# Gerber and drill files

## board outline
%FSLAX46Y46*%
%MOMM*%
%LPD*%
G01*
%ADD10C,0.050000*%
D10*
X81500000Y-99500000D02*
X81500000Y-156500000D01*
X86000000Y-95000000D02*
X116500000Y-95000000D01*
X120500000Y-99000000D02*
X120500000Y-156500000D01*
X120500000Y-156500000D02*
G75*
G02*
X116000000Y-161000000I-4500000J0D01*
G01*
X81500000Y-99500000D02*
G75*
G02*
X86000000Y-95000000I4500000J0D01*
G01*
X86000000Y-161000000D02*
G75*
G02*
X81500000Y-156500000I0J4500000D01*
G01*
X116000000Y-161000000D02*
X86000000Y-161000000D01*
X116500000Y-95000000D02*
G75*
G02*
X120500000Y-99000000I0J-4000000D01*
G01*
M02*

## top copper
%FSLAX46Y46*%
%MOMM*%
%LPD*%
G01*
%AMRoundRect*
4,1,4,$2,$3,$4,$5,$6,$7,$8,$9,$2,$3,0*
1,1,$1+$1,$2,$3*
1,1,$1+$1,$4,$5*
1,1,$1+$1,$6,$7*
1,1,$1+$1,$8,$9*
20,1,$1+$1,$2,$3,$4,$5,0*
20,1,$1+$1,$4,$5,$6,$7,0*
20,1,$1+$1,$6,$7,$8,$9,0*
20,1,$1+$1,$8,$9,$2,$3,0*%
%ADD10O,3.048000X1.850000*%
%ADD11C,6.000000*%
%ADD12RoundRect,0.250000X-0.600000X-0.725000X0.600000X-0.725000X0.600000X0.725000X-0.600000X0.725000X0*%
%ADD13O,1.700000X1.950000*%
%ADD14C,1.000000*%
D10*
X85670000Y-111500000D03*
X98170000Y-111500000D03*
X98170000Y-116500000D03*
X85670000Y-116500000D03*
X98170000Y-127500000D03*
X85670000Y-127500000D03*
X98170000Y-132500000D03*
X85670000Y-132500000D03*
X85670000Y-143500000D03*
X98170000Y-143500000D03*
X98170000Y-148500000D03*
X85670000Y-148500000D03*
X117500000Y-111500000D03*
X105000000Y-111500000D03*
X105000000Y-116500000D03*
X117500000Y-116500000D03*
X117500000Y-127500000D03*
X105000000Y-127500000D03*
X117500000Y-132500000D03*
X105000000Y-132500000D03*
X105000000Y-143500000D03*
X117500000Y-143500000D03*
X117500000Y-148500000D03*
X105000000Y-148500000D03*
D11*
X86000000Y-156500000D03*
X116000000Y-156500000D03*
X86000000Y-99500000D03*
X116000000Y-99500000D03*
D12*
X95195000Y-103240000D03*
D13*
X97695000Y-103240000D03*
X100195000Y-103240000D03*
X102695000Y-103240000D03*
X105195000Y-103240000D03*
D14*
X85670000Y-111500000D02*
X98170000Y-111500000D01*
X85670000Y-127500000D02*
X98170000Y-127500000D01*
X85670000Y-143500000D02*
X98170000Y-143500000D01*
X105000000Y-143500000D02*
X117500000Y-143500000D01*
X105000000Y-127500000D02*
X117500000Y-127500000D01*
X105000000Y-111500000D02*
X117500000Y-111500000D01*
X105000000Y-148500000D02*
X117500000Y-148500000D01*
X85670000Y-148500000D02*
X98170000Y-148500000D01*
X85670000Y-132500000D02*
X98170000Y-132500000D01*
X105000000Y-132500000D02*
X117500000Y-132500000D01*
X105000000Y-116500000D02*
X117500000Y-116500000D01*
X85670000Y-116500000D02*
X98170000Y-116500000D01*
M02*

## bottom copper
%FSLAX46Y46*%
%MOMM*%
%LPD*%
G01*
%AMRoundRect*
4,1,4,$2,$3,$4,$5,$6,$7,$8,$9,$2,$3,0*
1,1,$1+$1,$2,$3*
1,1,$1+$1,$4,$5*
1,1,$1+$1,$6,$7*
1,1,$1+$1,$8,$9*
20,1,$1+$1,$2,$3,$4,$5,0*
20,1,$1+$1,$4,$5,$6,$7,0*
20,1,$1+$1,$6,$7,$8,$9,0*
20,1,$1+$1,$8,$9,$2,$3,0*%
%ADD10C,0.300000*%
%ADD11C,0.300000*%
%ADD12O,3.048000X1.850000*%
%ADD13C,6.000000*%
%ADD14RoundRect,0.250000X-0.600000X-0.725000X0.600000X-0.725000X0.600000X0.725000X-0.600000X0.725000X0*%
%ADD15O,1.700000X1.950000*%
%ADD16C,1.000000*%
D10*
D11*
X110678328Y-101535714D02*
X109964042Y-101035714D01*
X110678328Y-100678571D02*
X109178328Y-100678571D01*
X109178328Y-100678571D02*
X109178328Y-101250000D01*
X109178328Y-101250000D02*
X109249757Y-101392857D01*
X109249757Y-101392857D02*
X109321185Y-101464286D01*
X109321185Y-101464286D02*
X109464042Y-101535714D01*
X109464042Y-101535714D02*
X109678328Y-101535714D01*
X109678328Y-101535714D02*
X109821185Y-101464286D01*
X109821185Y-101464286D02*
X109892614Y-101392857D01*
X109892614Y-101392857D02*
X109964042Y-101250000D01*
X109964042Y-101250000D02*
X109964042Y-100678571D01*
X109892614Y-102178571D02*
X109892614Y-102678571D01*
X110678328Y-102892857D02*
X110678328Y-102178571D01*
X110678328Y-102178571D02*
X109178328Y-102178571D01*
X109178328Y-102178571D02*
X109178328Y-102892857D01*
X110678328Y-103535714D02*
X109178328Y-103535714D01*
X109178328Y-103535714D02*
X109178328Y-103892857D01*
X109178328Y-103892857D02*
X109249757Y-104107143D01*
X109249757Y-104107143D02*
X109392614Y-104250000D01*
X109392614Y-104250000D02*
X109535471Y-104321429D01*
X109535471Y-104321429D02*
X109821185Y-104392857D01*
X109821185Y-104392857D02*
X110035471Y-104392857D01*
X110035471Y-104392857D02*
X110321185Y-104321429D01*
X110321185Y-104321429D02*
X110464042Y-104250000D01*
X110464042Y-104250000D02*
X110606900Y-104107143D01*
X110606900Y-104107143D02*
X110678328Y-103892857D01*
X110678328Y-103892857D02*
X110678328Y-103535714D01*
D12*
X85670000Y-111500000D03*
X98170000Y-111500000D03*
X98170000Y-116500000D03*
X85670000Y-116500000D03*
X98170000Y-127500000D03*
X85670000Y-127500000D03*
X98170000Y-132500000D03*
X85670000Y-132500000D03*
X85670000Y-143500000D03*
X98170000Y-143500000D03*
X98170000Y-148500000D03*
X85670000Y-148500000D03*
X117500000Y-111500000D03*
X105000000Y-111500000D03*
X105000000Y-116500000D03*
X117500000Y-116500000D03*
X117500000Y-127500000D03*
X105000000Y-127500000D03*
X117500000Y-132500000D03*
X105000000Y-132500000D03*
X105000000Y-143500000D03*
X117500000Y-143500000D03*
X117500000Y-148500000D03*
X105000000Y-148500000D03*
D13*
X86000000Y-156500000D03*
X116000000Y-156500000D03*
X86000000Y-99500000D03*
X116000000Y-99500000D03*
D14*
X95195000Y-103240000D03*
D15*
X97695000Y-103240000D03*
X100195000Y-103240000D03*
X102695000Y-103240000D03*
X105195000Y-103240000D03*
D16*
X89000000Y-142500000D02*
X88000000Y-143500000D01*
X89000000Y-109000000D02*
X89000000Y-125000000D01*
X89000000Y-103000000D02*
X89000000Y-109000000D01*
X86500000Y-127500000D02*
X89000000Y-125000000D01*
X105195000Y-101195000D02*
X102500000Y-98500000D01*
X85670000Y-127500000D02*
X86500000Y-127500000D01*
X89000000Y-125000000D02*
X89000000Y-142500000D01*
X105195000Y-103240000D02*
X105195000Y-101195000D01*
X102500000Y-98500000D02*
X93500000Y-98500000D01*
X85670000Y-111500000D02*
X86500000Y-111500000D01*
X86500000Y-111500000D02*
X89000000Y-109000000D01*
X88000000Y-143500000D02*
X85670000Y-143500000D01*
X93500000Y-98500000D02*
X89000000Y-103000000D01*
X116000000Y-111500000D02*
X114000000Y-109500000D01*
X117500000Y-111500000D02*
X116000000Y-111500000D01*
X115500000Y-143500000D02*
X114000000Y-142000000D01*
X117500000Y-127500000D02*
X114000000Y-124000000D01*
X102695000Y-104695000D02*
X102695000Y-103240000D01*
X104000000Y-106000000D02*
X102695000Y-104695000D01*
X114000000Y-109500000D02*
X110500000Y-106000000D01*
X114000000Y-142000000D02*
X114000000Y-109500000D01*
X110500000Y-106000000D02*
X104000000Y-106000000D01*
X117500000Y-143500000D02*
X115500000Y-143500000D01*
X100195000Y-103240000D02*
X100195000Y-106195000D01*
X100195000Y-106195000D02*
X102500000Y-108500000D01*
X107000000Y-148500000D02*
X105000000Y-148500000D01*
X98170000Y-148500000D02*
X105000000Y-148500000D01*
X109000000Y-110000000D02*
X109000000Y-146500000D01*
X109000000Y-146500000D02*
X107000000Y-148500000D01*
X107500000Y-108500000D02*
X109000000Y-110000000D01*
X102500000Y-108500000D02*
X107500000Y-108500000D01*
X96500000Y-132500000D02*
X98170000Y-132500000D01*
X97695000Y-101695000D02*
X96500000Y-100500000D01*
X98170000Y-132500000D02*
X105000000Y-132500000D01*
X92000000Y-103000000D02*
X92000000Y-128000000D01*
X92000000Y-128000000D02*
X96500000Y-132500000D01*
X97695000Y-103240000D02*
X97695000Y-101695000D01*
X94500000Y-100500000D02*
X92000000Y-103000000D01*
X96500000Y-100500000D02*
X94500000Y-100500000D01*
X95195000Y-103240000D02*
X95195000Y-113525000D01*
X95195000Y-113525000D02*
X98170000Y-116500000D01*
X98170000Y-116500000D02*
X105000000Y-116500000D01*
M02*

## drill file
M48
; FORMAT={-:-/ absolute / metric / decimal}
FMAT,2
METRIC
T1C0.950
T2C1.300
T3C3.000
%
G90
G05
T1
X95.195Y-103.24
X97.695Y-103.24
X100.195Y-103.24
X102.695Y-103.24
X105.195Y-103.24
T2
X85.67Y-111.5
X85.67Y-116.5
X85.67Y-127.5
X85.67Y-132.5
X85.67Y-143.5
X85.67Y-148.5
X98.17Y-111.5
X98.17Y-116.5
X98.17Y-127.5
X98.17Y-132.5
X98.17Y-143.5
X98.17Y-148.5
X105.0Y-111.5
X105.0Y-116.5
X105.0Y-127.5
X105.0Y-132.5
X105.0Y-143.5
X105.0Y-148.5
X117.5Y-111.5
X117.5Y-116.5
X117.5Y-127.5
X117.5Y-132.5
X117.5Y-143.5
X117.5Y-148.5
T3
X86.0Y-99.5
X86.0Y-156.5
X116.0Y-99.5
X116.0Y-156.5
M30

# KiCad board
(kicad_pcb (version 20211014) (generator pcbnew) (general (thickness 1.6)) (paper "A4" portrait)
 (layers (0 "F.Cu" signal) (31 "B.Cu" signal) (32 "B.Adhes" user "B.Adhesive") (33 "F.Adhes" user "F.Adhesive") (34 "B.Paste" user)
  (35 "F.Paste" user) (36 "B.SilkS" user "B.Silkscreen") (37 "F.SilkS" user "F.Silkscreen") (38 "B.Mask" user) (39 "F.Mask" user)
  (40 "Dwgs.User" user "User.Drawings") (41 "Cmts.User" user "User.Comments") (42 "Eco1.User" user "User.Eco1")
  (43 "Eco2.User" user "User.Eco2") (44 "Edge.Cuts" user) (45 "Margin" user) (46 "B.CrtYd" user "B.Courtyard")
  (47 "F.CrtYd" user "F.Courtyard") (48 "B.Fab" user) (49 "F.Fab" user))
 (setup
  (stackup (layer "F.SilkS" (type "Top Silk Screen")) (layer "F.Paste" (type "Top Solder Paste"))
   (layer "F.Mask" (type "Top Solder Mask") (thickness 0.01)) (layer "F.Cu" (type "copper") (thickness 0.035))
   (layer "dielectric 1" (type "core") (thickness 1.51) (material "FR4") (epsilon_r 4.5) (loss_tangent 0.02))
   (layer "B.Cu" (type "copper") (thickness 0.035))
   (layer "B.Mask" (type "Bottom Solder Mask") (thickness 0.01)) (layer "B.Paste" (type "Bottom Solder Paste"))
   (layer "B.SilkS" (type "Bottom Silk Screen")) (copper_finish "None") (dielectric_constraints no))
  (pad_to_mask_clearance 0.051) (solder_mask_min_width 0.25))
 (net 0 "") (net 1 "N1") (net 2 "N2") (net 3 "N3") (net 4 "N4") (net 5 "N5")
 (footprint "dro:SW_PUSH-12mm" (layer "F.Cu") (at 85.67 111.5)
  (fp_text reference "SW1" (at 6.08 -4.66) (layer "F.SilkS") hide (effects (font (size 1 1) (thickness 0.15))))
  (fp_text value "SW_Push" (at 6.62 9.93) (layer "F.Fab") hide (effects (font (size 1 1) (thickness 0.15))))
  (pad "1" thru_hole oval locked (at 0 0) (size 3.048 1.85) (drill 1.3) (layers *.Cu *.Mask) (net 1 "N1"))
  (pad "1" thru_hole oval locked (at 12.5 0) (size 3.048 1.85) (drill 1.3) (layers *.Cu *.Mask) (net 1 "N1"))
  (pad "2" thru_hole oval locked (at 12.5 5) (size 3.048 1.85) (drill 1.3) (layers *.Cu *.Mask) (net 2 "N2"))
  (pad "2" thru_hole oval locked (at 0 5) (size 3.048 1.85) (drill 1.3) (layers *.Cu *.Mask) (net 2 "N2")))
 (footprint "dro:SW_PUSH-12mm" (layer "F.Cu") (at 85.67 127.5)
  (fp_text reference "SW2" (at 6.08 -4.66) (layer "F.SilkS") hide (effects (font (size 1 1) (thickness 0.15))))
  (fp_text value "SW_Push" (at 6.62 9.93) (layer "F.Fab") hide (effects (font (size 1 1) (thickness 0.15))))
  (pad "1" thru_hole oval locked (at 12.5 0) (size 3.048 1.85) (drill 1.3) (layers *.Cu *.Mask) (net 1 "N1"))
  (pad "1" thru_hole oval locked (at 0 0) (size 3.048 1.85) (drill 1.3) (layers *.Cu *.Mask) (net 1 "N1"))
  (pad "2" thru_hole oval locked (at 12.5 5) (size 3.048 1.85) (drill 1.3) (layers *.Cu *.Mask) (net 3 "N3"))
  (pad "2" thru_hole oval locked (at 0 5) (size 3.048 1.85) (drill 1.3) (layers *.Cu *.Mask) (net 3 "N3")))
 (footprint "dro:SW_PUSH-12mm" (layer "F.Cu") (at 85.67 143.5)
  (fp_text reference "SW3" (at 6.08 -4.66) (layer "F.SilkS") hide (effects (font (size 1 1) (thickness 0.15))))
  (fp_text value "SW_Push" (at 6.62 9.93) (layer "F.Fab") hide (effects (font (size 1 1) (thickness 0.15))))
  (pad "1" thru_hole oval locked (at 0 0) (size 3.048 1.85) (drill 1.3) (layers *.Cu *.Mask) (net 1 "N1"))
  (pad "1" thru_hole oval locked (at 12.5 0) (size 3.048 1.85) (drill 1.3) (layers *.Cu *.Mask) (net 1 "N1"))
  (pad "2" thru_hole oval locked (at 12.5 5) (size 3.048 1.85) (drill 1.3) (layers *.Cu *.Mask) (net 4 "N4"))
  (pad "2" thru_hole oval locked (at 0 5) (size 3.048 1.85) (drill 1.3) (layers *.Cu *.Mask) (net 4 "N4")))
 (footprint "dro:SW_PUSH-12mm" (layer "F.Cu") (at 105 111.5)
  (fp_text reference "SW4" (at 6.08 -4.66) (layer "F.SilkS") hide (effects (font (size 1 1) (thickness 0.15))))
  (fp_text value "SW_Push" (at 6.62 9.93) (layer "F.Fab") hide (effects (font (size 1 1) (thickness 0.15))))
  (pad "1" thru_hole oval locked (at 12.5 0) (size 3.048 1.85) (drill 1.3) (layers *.Cu *.Mask) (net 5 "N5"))
  (pad "1" thru_hole oval locked (at 0 0) (size 3.048 1.85) (drill 1.3) (layers *.Cu *.Mask) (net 5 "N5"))
  (pad "2" thru_hole oval locked (at 0 5) (size 3.048 1.85) (drill 1.3) (layers *.Cu *.Mask) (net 2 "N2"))
  (pad "2" thru_hole oval locked (at 12.5 5) (size 3.048 1.85) (drill 1.3) (layers *.Cu *.Mask) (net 2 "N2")))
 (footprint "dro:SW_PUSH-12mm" (layer "F.Cu") (at 105 127.5)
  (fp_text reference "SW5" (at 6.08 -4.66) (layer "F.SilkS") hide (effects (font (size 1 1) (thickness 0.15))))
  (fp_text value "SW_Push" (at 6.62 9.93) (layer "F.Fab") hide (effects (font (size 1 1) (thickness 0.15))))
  (pad "1" thru_hole oval locked (at 12.5 0) (size 3.048 1.85) (drill 1.3) (layers *.Cu *.Mask) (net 5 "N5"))
  (pad "1" thru_hole oval locked (at 0 0) (size 3.048 1.85) (drill 1.3) (layers *.Cu *.Mask) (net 5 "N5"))
  (pad "2" thru_hole oval locked (at 12.5 5) (size 3.048 1.85) (drill 1.3) (layers *.Cu *.Mask) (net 3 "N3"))
  (pad "2" thru_hole oval locked (at 0 5) (size 3.048 1.85) (drill 1.3) (layers *.Cu *.Mask) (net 3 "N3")))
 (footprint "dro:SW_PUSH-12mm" (layer "F.Cu") (at 105 143.5)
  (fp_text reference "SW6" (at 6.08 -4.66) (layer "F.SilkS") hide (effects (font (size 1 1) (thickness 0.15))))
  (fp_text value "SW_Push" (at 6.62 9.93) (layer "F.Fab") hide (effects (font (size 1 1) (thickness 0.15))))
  (pad "1" thru_hole oval locked (at 0 0) (size 3.048 1.85) (drill 1.3) (layers *.Cu *.Mask) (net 5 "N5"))
  (pad "1" thru_hole oval locked (at 12.5 0) (size 3.048 1.85) (drill 1.3) (layers *.Cu *.Mask) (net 5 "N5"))
  (pad "2" thru_hole oval locked (at 12.5 5) (size 3.048 1.85) (drill 1.3) (layers *.Cu *.Mask) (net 4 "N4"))
  (pad "2" thru_hole oval locked (at 0 5) (size 3.048 1.85) (drill 1.3) (layers *.Cu *.Mask) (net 4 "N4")))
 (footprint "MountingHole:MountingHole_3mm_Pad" (layer "F.Cu") (at 86 156.5)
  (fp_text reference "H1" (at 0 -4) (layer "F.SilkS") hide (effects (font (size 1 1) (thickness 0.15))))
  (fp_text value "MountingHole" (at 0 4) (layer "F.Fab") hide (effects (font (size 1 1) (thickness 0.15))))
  (pad "1" thru_hole circle locked (at 0 0) (size 6 6) (drill 3) (layers *.Cu *.Mask)))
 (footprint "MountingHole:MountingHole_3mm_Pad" (layer "F.Cu") (at 116 156.5)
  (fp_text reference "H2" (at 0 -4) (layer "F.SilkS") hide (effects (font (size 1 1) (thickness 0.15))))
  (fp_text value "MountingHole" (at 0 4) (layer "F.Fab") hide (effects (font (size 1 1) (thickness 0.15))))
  (pad "1" thru_hole circle locked (at 0 0) (size 6 6) (drill 3) (layers *.Cu *.Mask)))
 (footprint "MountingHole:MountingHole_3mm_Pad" (layer "F.Cu") (at 86 99.5)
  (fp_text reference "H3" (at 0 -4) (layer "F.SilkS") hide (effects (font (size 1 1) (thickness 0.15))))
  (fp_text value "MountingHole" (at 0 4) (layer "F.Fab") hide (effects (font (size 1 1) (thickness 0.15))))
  (pad "1" thru_hole circle locked (at 0 0) (size 6 6) (drill 3) (layers *.Cu *.Mask)))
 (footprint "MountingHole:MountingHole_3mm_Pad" (layer "F.Cu") (at 116 99.5)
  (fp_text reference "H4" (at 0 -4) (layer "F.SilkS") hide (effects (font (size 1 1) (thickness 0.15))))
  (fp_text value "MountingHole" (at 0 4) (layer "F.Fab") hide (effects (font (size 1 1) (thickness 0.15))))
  (pad "1" thru_hole circle locked (at 0 0) (size 6 6) (drill 3) (layers *.Cu *.Mask)))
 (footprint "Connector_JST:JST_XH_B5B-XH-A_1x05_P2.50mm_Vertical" (layer "B.Cu") (at 95.195 103.24)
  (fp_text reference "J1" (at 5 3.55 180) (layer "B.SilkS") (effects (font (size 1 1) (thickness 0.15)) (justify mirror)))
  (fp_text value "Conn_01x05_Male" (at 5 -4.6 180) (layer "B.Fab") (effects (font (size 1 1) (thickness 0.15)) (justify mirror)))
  (pad "1" thru_hole roundrect (at 0 0) (size 1.7 1.95) (drill 0.95) (layers *.Cu *.Mask) (roundrect_rratio 0.147059) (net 2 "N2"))
  (pad "2" thru_hole oval (at 2.5 0) (size 1.7 1.95) (drill 0.95) (layers *.Cu *.Mask) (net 3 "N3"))
  (pad "3" thru_hole oval (at 5 0) (size 1.7 1.95) (drill 0.95) (layers *.Cu *.Mask) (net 4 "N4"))
  (pad "4" thru_hole oval (at 7.5 0) (size 1.7 1.95) (drill 0.95) (layers *.Cu *.Mask) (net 5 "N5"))
  (pad "5" thru_hole oval (at 10 0) (size 1.7 1.95) (drill 0.95) (layers *.Cu *.Mask) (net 1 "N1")))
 (gr_line (start 81.5 99.5) (end 81.5 156.5) (layer "Edge.Cuts") (width 0.05))
 (gr_line (start 86 95) (end 116.5 95) (layer "Edge.Cuts") (width 0.05))
 (gr_line (start 120.5 99) (end 120.5 156.5) (layer "Edge.Cuts") (width 0.05))
 (gr_arc (start 120.5 156.5) (mid 119.181981 159.681981) (end 116 161) (layer "Edge.Cuts") (width 0.05))
 (gr_arc (start 81.5 99.5) (mid 82.818019 96.318019) (end 86 95) (layer "Edge.Cuts") (width 0.05))
 (gr_arc (start 86 161) (mid 82.818019 159.681981) (end 81.5 156.5) (layer "Edge.Cuts") (width 0.05))
 (gr_line (start 116 161) (end 86 161) (layer "Edge.Cuts") (width 0.05))
 (gr_arc (start 116.5 95) (mid 119.328427 96.171573) (end 120.5 99) (layer "Edge.Cuts") (width 0.05))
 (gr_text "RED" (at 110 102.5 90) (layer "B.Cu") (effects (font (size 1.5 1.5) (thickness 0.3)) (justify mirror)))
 (segment (start 85.67 111.5) (end 98.17 111.5) (width 1) (layer "F.Cu") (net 1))
 (segment (start 85.67 127.5) (end 98.17 127.5) (width 1) (layer "F.Cu") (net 1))
 (segment (start 85.67 143.5) (end 98.17 143.5) (width 1) (layer "F.Cu") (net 1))
 (segment (start 89 142.5) (end 88 143.5) (width 1) (layer "B.Cu") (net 1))
 (segment (start 89 109) (end 89 125) (width 1) (layer "B.Cu") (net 1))
 (segment (start 89 103) (end 89 109) (width 1) (layer "B.Cu") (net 1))
 (segment (start 86.5 127.5) (end 89 125) (width 1) (layer "B.Cu") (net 1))
 (segment (start 105.195 101.195) (end 102.5 98.5) (width 1) (layer "B.Cu") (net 1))
 (segment (start 85.67 127.5) (end 86.5 127.5) (width 1) (layer "B.Cu") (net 1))
 (segment (start 89 125) (end 89 142.5) (width 1) (layer "B.Cu") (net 1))
 (segment (start 105.195 103.24) (end 105.195 101.195) (width 1) (layer "B.Cu") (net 1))
 (segment (start 102.5 98.5) (end 93.5 98.5) (width 1) (layer "B.Cu") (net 1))
 (segment (start 85.67 111.5) (end 86.5 111.5) (width 1) (layer "B.Cu") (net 1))
 (segment (start 86.5 111.5) (end 89 109) (width 1) (layer "B.Cu") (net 1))
 (segment (start 88 143.5) (end 85.67 143.5) (width 1) (layer "B.Cu") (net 1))
 (segment (start 93.5 98.5) (end 89 103) (width 1) (layer "B.Cu") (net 1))
 (segment (start 105 143.5) (end 117.5 143.5) (width 1) (layer "F.Cu") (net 5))
 (segment (start 105 127.5) (end 117.5 127.5) (width 1) (layer "F.Cu") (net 5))
 (segment (start 105 111.5) (end 117.5 111.5) (width 1) (layer "F.Cu") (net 5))
 (segment (start 116 111.5) (end 114 109.5) (width 1) (layer "B.Cu") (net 5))
 (segment (start 117.5 111.5) (end 116 111.5) (width 1) (layer "B.Cu") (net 5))
 (segment (start 115.5 143.5) (end 114 142) (width 1) (layer "B.Cu") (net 5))
 (segment (start 117.5 127.5) (end 114 124) (width 1) (layer "B.Cu") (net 5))
 (segment (start 102.695 104.695) (end 102.695 103.24) (width 1) (layer "B.Cu") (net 5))
 (segment (start 104 106) (end 102.695 104.695) (width 1) (layer "B.Cu") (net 5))
 (segment (start 114 109.5) (end 110.5 106) (width 1) (layer "B.Cu") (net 5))
 (segment (start 114 142) (end 114 109.5) (width 1) (layer "B.Cu") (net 5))
 (segment (start 110.5 106) (end 104 106) (width 1) (layer "B.Cu") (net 5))
 (segment (start 117.5 143.5) (end 115.5 143.5) (width 1) (layer "B.Cu") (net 5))
 (segment (start 105 148.5) (end 117.5 148.5) (width 1) (layer "F.Cu") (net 4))
 (segment (start 85.67 148.5) (end 98.17 148.5) (width 1) (layer "F.Cu") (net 4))
 (segment (start 100.195 103.24) (end 100.195 106.195) (width 1) (layer "B.Cu") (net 4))
 (segment (start 100.195 106.195) (end 102.5 108.5) (width 1) (layer "B.Cu") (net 4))
 (segment (start 107 148.5) (end 105 148.5) (width 1) (layer "B.Cu") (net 4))
 (segment (start 98.17 148.5) (end 105 148.5) (width 1) (layer "B.Cu") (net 4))
 (segment (start 109 110) (end 109 146.5) (width 1) (layer "B.Cu") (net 4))
 (segment (start 109 146.5) (end 107 148.5) (width 1) (layer "B.Cu") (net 4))
 (segment (start 107.5 108.5) (end 109 110) (width 1) (layer "B.Cu") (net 4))
 (segment (start 102.5 108.5) (end 107.5 108.5) (width 1) (layer "B.Cu") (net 4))
 (segment (start 85.67 132.5) (end 98.17 132.5) (width 1) (layer "F.Cu") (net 3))
 (segment (start 105 132.5) (end 117.5 132.5) (width 1) (layer "F.Cu") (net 3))
 (segment (start 96.5 132.5) (end 98.17 132.5) (width 1) (layer "B.Cu") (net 3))
 (segment (start 97.695 101.695) (end 96.5 100.5) (width 1) (layer "B.Cu") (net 3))
 (segment (start 98.17 132.5) (end 105 132.5) (width 1) (layer "B.Cu") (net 3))
 (segment (start 92 103) (end 92 128) (width 1) (layer "B.Cu") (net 3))
 (segment (start 92 128) (end 96.5 132.5) (width 1) (layer "B.Cu") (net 3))
 (segment (start 97.695 103.24) (end 97.695 101.695) (width 1) (layer "B.Cu") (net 3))
 (segment (start 94.5 100.5) (end 92 103) (width 1) (layer "B.Cu") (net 3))
 (segment (start 96.5 100.5) (end 94.5 100.5) (width 1) (layer "B.Cu") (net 3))
 (segment (start 105 116.5) (end 117.5 116.5) (width 1) (layer "F.Cu") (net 2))
 (segment (start 85.67 116.5) (end 98.17 116.5) (width 1) (layer "F.Cu") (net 2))
 (segment (start 95.195 103.24) (end 95.195 113.525) (width 1) (layer "B.Cu") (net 2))
 (segment (start 95.195 113.525) (end 98.17 116.5) (width 1) (layer "B.Cu") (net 2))
 (segment (start 98.17 116.5) (end 105 116.5) (width 1) (layer "B.Cu") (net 2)))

